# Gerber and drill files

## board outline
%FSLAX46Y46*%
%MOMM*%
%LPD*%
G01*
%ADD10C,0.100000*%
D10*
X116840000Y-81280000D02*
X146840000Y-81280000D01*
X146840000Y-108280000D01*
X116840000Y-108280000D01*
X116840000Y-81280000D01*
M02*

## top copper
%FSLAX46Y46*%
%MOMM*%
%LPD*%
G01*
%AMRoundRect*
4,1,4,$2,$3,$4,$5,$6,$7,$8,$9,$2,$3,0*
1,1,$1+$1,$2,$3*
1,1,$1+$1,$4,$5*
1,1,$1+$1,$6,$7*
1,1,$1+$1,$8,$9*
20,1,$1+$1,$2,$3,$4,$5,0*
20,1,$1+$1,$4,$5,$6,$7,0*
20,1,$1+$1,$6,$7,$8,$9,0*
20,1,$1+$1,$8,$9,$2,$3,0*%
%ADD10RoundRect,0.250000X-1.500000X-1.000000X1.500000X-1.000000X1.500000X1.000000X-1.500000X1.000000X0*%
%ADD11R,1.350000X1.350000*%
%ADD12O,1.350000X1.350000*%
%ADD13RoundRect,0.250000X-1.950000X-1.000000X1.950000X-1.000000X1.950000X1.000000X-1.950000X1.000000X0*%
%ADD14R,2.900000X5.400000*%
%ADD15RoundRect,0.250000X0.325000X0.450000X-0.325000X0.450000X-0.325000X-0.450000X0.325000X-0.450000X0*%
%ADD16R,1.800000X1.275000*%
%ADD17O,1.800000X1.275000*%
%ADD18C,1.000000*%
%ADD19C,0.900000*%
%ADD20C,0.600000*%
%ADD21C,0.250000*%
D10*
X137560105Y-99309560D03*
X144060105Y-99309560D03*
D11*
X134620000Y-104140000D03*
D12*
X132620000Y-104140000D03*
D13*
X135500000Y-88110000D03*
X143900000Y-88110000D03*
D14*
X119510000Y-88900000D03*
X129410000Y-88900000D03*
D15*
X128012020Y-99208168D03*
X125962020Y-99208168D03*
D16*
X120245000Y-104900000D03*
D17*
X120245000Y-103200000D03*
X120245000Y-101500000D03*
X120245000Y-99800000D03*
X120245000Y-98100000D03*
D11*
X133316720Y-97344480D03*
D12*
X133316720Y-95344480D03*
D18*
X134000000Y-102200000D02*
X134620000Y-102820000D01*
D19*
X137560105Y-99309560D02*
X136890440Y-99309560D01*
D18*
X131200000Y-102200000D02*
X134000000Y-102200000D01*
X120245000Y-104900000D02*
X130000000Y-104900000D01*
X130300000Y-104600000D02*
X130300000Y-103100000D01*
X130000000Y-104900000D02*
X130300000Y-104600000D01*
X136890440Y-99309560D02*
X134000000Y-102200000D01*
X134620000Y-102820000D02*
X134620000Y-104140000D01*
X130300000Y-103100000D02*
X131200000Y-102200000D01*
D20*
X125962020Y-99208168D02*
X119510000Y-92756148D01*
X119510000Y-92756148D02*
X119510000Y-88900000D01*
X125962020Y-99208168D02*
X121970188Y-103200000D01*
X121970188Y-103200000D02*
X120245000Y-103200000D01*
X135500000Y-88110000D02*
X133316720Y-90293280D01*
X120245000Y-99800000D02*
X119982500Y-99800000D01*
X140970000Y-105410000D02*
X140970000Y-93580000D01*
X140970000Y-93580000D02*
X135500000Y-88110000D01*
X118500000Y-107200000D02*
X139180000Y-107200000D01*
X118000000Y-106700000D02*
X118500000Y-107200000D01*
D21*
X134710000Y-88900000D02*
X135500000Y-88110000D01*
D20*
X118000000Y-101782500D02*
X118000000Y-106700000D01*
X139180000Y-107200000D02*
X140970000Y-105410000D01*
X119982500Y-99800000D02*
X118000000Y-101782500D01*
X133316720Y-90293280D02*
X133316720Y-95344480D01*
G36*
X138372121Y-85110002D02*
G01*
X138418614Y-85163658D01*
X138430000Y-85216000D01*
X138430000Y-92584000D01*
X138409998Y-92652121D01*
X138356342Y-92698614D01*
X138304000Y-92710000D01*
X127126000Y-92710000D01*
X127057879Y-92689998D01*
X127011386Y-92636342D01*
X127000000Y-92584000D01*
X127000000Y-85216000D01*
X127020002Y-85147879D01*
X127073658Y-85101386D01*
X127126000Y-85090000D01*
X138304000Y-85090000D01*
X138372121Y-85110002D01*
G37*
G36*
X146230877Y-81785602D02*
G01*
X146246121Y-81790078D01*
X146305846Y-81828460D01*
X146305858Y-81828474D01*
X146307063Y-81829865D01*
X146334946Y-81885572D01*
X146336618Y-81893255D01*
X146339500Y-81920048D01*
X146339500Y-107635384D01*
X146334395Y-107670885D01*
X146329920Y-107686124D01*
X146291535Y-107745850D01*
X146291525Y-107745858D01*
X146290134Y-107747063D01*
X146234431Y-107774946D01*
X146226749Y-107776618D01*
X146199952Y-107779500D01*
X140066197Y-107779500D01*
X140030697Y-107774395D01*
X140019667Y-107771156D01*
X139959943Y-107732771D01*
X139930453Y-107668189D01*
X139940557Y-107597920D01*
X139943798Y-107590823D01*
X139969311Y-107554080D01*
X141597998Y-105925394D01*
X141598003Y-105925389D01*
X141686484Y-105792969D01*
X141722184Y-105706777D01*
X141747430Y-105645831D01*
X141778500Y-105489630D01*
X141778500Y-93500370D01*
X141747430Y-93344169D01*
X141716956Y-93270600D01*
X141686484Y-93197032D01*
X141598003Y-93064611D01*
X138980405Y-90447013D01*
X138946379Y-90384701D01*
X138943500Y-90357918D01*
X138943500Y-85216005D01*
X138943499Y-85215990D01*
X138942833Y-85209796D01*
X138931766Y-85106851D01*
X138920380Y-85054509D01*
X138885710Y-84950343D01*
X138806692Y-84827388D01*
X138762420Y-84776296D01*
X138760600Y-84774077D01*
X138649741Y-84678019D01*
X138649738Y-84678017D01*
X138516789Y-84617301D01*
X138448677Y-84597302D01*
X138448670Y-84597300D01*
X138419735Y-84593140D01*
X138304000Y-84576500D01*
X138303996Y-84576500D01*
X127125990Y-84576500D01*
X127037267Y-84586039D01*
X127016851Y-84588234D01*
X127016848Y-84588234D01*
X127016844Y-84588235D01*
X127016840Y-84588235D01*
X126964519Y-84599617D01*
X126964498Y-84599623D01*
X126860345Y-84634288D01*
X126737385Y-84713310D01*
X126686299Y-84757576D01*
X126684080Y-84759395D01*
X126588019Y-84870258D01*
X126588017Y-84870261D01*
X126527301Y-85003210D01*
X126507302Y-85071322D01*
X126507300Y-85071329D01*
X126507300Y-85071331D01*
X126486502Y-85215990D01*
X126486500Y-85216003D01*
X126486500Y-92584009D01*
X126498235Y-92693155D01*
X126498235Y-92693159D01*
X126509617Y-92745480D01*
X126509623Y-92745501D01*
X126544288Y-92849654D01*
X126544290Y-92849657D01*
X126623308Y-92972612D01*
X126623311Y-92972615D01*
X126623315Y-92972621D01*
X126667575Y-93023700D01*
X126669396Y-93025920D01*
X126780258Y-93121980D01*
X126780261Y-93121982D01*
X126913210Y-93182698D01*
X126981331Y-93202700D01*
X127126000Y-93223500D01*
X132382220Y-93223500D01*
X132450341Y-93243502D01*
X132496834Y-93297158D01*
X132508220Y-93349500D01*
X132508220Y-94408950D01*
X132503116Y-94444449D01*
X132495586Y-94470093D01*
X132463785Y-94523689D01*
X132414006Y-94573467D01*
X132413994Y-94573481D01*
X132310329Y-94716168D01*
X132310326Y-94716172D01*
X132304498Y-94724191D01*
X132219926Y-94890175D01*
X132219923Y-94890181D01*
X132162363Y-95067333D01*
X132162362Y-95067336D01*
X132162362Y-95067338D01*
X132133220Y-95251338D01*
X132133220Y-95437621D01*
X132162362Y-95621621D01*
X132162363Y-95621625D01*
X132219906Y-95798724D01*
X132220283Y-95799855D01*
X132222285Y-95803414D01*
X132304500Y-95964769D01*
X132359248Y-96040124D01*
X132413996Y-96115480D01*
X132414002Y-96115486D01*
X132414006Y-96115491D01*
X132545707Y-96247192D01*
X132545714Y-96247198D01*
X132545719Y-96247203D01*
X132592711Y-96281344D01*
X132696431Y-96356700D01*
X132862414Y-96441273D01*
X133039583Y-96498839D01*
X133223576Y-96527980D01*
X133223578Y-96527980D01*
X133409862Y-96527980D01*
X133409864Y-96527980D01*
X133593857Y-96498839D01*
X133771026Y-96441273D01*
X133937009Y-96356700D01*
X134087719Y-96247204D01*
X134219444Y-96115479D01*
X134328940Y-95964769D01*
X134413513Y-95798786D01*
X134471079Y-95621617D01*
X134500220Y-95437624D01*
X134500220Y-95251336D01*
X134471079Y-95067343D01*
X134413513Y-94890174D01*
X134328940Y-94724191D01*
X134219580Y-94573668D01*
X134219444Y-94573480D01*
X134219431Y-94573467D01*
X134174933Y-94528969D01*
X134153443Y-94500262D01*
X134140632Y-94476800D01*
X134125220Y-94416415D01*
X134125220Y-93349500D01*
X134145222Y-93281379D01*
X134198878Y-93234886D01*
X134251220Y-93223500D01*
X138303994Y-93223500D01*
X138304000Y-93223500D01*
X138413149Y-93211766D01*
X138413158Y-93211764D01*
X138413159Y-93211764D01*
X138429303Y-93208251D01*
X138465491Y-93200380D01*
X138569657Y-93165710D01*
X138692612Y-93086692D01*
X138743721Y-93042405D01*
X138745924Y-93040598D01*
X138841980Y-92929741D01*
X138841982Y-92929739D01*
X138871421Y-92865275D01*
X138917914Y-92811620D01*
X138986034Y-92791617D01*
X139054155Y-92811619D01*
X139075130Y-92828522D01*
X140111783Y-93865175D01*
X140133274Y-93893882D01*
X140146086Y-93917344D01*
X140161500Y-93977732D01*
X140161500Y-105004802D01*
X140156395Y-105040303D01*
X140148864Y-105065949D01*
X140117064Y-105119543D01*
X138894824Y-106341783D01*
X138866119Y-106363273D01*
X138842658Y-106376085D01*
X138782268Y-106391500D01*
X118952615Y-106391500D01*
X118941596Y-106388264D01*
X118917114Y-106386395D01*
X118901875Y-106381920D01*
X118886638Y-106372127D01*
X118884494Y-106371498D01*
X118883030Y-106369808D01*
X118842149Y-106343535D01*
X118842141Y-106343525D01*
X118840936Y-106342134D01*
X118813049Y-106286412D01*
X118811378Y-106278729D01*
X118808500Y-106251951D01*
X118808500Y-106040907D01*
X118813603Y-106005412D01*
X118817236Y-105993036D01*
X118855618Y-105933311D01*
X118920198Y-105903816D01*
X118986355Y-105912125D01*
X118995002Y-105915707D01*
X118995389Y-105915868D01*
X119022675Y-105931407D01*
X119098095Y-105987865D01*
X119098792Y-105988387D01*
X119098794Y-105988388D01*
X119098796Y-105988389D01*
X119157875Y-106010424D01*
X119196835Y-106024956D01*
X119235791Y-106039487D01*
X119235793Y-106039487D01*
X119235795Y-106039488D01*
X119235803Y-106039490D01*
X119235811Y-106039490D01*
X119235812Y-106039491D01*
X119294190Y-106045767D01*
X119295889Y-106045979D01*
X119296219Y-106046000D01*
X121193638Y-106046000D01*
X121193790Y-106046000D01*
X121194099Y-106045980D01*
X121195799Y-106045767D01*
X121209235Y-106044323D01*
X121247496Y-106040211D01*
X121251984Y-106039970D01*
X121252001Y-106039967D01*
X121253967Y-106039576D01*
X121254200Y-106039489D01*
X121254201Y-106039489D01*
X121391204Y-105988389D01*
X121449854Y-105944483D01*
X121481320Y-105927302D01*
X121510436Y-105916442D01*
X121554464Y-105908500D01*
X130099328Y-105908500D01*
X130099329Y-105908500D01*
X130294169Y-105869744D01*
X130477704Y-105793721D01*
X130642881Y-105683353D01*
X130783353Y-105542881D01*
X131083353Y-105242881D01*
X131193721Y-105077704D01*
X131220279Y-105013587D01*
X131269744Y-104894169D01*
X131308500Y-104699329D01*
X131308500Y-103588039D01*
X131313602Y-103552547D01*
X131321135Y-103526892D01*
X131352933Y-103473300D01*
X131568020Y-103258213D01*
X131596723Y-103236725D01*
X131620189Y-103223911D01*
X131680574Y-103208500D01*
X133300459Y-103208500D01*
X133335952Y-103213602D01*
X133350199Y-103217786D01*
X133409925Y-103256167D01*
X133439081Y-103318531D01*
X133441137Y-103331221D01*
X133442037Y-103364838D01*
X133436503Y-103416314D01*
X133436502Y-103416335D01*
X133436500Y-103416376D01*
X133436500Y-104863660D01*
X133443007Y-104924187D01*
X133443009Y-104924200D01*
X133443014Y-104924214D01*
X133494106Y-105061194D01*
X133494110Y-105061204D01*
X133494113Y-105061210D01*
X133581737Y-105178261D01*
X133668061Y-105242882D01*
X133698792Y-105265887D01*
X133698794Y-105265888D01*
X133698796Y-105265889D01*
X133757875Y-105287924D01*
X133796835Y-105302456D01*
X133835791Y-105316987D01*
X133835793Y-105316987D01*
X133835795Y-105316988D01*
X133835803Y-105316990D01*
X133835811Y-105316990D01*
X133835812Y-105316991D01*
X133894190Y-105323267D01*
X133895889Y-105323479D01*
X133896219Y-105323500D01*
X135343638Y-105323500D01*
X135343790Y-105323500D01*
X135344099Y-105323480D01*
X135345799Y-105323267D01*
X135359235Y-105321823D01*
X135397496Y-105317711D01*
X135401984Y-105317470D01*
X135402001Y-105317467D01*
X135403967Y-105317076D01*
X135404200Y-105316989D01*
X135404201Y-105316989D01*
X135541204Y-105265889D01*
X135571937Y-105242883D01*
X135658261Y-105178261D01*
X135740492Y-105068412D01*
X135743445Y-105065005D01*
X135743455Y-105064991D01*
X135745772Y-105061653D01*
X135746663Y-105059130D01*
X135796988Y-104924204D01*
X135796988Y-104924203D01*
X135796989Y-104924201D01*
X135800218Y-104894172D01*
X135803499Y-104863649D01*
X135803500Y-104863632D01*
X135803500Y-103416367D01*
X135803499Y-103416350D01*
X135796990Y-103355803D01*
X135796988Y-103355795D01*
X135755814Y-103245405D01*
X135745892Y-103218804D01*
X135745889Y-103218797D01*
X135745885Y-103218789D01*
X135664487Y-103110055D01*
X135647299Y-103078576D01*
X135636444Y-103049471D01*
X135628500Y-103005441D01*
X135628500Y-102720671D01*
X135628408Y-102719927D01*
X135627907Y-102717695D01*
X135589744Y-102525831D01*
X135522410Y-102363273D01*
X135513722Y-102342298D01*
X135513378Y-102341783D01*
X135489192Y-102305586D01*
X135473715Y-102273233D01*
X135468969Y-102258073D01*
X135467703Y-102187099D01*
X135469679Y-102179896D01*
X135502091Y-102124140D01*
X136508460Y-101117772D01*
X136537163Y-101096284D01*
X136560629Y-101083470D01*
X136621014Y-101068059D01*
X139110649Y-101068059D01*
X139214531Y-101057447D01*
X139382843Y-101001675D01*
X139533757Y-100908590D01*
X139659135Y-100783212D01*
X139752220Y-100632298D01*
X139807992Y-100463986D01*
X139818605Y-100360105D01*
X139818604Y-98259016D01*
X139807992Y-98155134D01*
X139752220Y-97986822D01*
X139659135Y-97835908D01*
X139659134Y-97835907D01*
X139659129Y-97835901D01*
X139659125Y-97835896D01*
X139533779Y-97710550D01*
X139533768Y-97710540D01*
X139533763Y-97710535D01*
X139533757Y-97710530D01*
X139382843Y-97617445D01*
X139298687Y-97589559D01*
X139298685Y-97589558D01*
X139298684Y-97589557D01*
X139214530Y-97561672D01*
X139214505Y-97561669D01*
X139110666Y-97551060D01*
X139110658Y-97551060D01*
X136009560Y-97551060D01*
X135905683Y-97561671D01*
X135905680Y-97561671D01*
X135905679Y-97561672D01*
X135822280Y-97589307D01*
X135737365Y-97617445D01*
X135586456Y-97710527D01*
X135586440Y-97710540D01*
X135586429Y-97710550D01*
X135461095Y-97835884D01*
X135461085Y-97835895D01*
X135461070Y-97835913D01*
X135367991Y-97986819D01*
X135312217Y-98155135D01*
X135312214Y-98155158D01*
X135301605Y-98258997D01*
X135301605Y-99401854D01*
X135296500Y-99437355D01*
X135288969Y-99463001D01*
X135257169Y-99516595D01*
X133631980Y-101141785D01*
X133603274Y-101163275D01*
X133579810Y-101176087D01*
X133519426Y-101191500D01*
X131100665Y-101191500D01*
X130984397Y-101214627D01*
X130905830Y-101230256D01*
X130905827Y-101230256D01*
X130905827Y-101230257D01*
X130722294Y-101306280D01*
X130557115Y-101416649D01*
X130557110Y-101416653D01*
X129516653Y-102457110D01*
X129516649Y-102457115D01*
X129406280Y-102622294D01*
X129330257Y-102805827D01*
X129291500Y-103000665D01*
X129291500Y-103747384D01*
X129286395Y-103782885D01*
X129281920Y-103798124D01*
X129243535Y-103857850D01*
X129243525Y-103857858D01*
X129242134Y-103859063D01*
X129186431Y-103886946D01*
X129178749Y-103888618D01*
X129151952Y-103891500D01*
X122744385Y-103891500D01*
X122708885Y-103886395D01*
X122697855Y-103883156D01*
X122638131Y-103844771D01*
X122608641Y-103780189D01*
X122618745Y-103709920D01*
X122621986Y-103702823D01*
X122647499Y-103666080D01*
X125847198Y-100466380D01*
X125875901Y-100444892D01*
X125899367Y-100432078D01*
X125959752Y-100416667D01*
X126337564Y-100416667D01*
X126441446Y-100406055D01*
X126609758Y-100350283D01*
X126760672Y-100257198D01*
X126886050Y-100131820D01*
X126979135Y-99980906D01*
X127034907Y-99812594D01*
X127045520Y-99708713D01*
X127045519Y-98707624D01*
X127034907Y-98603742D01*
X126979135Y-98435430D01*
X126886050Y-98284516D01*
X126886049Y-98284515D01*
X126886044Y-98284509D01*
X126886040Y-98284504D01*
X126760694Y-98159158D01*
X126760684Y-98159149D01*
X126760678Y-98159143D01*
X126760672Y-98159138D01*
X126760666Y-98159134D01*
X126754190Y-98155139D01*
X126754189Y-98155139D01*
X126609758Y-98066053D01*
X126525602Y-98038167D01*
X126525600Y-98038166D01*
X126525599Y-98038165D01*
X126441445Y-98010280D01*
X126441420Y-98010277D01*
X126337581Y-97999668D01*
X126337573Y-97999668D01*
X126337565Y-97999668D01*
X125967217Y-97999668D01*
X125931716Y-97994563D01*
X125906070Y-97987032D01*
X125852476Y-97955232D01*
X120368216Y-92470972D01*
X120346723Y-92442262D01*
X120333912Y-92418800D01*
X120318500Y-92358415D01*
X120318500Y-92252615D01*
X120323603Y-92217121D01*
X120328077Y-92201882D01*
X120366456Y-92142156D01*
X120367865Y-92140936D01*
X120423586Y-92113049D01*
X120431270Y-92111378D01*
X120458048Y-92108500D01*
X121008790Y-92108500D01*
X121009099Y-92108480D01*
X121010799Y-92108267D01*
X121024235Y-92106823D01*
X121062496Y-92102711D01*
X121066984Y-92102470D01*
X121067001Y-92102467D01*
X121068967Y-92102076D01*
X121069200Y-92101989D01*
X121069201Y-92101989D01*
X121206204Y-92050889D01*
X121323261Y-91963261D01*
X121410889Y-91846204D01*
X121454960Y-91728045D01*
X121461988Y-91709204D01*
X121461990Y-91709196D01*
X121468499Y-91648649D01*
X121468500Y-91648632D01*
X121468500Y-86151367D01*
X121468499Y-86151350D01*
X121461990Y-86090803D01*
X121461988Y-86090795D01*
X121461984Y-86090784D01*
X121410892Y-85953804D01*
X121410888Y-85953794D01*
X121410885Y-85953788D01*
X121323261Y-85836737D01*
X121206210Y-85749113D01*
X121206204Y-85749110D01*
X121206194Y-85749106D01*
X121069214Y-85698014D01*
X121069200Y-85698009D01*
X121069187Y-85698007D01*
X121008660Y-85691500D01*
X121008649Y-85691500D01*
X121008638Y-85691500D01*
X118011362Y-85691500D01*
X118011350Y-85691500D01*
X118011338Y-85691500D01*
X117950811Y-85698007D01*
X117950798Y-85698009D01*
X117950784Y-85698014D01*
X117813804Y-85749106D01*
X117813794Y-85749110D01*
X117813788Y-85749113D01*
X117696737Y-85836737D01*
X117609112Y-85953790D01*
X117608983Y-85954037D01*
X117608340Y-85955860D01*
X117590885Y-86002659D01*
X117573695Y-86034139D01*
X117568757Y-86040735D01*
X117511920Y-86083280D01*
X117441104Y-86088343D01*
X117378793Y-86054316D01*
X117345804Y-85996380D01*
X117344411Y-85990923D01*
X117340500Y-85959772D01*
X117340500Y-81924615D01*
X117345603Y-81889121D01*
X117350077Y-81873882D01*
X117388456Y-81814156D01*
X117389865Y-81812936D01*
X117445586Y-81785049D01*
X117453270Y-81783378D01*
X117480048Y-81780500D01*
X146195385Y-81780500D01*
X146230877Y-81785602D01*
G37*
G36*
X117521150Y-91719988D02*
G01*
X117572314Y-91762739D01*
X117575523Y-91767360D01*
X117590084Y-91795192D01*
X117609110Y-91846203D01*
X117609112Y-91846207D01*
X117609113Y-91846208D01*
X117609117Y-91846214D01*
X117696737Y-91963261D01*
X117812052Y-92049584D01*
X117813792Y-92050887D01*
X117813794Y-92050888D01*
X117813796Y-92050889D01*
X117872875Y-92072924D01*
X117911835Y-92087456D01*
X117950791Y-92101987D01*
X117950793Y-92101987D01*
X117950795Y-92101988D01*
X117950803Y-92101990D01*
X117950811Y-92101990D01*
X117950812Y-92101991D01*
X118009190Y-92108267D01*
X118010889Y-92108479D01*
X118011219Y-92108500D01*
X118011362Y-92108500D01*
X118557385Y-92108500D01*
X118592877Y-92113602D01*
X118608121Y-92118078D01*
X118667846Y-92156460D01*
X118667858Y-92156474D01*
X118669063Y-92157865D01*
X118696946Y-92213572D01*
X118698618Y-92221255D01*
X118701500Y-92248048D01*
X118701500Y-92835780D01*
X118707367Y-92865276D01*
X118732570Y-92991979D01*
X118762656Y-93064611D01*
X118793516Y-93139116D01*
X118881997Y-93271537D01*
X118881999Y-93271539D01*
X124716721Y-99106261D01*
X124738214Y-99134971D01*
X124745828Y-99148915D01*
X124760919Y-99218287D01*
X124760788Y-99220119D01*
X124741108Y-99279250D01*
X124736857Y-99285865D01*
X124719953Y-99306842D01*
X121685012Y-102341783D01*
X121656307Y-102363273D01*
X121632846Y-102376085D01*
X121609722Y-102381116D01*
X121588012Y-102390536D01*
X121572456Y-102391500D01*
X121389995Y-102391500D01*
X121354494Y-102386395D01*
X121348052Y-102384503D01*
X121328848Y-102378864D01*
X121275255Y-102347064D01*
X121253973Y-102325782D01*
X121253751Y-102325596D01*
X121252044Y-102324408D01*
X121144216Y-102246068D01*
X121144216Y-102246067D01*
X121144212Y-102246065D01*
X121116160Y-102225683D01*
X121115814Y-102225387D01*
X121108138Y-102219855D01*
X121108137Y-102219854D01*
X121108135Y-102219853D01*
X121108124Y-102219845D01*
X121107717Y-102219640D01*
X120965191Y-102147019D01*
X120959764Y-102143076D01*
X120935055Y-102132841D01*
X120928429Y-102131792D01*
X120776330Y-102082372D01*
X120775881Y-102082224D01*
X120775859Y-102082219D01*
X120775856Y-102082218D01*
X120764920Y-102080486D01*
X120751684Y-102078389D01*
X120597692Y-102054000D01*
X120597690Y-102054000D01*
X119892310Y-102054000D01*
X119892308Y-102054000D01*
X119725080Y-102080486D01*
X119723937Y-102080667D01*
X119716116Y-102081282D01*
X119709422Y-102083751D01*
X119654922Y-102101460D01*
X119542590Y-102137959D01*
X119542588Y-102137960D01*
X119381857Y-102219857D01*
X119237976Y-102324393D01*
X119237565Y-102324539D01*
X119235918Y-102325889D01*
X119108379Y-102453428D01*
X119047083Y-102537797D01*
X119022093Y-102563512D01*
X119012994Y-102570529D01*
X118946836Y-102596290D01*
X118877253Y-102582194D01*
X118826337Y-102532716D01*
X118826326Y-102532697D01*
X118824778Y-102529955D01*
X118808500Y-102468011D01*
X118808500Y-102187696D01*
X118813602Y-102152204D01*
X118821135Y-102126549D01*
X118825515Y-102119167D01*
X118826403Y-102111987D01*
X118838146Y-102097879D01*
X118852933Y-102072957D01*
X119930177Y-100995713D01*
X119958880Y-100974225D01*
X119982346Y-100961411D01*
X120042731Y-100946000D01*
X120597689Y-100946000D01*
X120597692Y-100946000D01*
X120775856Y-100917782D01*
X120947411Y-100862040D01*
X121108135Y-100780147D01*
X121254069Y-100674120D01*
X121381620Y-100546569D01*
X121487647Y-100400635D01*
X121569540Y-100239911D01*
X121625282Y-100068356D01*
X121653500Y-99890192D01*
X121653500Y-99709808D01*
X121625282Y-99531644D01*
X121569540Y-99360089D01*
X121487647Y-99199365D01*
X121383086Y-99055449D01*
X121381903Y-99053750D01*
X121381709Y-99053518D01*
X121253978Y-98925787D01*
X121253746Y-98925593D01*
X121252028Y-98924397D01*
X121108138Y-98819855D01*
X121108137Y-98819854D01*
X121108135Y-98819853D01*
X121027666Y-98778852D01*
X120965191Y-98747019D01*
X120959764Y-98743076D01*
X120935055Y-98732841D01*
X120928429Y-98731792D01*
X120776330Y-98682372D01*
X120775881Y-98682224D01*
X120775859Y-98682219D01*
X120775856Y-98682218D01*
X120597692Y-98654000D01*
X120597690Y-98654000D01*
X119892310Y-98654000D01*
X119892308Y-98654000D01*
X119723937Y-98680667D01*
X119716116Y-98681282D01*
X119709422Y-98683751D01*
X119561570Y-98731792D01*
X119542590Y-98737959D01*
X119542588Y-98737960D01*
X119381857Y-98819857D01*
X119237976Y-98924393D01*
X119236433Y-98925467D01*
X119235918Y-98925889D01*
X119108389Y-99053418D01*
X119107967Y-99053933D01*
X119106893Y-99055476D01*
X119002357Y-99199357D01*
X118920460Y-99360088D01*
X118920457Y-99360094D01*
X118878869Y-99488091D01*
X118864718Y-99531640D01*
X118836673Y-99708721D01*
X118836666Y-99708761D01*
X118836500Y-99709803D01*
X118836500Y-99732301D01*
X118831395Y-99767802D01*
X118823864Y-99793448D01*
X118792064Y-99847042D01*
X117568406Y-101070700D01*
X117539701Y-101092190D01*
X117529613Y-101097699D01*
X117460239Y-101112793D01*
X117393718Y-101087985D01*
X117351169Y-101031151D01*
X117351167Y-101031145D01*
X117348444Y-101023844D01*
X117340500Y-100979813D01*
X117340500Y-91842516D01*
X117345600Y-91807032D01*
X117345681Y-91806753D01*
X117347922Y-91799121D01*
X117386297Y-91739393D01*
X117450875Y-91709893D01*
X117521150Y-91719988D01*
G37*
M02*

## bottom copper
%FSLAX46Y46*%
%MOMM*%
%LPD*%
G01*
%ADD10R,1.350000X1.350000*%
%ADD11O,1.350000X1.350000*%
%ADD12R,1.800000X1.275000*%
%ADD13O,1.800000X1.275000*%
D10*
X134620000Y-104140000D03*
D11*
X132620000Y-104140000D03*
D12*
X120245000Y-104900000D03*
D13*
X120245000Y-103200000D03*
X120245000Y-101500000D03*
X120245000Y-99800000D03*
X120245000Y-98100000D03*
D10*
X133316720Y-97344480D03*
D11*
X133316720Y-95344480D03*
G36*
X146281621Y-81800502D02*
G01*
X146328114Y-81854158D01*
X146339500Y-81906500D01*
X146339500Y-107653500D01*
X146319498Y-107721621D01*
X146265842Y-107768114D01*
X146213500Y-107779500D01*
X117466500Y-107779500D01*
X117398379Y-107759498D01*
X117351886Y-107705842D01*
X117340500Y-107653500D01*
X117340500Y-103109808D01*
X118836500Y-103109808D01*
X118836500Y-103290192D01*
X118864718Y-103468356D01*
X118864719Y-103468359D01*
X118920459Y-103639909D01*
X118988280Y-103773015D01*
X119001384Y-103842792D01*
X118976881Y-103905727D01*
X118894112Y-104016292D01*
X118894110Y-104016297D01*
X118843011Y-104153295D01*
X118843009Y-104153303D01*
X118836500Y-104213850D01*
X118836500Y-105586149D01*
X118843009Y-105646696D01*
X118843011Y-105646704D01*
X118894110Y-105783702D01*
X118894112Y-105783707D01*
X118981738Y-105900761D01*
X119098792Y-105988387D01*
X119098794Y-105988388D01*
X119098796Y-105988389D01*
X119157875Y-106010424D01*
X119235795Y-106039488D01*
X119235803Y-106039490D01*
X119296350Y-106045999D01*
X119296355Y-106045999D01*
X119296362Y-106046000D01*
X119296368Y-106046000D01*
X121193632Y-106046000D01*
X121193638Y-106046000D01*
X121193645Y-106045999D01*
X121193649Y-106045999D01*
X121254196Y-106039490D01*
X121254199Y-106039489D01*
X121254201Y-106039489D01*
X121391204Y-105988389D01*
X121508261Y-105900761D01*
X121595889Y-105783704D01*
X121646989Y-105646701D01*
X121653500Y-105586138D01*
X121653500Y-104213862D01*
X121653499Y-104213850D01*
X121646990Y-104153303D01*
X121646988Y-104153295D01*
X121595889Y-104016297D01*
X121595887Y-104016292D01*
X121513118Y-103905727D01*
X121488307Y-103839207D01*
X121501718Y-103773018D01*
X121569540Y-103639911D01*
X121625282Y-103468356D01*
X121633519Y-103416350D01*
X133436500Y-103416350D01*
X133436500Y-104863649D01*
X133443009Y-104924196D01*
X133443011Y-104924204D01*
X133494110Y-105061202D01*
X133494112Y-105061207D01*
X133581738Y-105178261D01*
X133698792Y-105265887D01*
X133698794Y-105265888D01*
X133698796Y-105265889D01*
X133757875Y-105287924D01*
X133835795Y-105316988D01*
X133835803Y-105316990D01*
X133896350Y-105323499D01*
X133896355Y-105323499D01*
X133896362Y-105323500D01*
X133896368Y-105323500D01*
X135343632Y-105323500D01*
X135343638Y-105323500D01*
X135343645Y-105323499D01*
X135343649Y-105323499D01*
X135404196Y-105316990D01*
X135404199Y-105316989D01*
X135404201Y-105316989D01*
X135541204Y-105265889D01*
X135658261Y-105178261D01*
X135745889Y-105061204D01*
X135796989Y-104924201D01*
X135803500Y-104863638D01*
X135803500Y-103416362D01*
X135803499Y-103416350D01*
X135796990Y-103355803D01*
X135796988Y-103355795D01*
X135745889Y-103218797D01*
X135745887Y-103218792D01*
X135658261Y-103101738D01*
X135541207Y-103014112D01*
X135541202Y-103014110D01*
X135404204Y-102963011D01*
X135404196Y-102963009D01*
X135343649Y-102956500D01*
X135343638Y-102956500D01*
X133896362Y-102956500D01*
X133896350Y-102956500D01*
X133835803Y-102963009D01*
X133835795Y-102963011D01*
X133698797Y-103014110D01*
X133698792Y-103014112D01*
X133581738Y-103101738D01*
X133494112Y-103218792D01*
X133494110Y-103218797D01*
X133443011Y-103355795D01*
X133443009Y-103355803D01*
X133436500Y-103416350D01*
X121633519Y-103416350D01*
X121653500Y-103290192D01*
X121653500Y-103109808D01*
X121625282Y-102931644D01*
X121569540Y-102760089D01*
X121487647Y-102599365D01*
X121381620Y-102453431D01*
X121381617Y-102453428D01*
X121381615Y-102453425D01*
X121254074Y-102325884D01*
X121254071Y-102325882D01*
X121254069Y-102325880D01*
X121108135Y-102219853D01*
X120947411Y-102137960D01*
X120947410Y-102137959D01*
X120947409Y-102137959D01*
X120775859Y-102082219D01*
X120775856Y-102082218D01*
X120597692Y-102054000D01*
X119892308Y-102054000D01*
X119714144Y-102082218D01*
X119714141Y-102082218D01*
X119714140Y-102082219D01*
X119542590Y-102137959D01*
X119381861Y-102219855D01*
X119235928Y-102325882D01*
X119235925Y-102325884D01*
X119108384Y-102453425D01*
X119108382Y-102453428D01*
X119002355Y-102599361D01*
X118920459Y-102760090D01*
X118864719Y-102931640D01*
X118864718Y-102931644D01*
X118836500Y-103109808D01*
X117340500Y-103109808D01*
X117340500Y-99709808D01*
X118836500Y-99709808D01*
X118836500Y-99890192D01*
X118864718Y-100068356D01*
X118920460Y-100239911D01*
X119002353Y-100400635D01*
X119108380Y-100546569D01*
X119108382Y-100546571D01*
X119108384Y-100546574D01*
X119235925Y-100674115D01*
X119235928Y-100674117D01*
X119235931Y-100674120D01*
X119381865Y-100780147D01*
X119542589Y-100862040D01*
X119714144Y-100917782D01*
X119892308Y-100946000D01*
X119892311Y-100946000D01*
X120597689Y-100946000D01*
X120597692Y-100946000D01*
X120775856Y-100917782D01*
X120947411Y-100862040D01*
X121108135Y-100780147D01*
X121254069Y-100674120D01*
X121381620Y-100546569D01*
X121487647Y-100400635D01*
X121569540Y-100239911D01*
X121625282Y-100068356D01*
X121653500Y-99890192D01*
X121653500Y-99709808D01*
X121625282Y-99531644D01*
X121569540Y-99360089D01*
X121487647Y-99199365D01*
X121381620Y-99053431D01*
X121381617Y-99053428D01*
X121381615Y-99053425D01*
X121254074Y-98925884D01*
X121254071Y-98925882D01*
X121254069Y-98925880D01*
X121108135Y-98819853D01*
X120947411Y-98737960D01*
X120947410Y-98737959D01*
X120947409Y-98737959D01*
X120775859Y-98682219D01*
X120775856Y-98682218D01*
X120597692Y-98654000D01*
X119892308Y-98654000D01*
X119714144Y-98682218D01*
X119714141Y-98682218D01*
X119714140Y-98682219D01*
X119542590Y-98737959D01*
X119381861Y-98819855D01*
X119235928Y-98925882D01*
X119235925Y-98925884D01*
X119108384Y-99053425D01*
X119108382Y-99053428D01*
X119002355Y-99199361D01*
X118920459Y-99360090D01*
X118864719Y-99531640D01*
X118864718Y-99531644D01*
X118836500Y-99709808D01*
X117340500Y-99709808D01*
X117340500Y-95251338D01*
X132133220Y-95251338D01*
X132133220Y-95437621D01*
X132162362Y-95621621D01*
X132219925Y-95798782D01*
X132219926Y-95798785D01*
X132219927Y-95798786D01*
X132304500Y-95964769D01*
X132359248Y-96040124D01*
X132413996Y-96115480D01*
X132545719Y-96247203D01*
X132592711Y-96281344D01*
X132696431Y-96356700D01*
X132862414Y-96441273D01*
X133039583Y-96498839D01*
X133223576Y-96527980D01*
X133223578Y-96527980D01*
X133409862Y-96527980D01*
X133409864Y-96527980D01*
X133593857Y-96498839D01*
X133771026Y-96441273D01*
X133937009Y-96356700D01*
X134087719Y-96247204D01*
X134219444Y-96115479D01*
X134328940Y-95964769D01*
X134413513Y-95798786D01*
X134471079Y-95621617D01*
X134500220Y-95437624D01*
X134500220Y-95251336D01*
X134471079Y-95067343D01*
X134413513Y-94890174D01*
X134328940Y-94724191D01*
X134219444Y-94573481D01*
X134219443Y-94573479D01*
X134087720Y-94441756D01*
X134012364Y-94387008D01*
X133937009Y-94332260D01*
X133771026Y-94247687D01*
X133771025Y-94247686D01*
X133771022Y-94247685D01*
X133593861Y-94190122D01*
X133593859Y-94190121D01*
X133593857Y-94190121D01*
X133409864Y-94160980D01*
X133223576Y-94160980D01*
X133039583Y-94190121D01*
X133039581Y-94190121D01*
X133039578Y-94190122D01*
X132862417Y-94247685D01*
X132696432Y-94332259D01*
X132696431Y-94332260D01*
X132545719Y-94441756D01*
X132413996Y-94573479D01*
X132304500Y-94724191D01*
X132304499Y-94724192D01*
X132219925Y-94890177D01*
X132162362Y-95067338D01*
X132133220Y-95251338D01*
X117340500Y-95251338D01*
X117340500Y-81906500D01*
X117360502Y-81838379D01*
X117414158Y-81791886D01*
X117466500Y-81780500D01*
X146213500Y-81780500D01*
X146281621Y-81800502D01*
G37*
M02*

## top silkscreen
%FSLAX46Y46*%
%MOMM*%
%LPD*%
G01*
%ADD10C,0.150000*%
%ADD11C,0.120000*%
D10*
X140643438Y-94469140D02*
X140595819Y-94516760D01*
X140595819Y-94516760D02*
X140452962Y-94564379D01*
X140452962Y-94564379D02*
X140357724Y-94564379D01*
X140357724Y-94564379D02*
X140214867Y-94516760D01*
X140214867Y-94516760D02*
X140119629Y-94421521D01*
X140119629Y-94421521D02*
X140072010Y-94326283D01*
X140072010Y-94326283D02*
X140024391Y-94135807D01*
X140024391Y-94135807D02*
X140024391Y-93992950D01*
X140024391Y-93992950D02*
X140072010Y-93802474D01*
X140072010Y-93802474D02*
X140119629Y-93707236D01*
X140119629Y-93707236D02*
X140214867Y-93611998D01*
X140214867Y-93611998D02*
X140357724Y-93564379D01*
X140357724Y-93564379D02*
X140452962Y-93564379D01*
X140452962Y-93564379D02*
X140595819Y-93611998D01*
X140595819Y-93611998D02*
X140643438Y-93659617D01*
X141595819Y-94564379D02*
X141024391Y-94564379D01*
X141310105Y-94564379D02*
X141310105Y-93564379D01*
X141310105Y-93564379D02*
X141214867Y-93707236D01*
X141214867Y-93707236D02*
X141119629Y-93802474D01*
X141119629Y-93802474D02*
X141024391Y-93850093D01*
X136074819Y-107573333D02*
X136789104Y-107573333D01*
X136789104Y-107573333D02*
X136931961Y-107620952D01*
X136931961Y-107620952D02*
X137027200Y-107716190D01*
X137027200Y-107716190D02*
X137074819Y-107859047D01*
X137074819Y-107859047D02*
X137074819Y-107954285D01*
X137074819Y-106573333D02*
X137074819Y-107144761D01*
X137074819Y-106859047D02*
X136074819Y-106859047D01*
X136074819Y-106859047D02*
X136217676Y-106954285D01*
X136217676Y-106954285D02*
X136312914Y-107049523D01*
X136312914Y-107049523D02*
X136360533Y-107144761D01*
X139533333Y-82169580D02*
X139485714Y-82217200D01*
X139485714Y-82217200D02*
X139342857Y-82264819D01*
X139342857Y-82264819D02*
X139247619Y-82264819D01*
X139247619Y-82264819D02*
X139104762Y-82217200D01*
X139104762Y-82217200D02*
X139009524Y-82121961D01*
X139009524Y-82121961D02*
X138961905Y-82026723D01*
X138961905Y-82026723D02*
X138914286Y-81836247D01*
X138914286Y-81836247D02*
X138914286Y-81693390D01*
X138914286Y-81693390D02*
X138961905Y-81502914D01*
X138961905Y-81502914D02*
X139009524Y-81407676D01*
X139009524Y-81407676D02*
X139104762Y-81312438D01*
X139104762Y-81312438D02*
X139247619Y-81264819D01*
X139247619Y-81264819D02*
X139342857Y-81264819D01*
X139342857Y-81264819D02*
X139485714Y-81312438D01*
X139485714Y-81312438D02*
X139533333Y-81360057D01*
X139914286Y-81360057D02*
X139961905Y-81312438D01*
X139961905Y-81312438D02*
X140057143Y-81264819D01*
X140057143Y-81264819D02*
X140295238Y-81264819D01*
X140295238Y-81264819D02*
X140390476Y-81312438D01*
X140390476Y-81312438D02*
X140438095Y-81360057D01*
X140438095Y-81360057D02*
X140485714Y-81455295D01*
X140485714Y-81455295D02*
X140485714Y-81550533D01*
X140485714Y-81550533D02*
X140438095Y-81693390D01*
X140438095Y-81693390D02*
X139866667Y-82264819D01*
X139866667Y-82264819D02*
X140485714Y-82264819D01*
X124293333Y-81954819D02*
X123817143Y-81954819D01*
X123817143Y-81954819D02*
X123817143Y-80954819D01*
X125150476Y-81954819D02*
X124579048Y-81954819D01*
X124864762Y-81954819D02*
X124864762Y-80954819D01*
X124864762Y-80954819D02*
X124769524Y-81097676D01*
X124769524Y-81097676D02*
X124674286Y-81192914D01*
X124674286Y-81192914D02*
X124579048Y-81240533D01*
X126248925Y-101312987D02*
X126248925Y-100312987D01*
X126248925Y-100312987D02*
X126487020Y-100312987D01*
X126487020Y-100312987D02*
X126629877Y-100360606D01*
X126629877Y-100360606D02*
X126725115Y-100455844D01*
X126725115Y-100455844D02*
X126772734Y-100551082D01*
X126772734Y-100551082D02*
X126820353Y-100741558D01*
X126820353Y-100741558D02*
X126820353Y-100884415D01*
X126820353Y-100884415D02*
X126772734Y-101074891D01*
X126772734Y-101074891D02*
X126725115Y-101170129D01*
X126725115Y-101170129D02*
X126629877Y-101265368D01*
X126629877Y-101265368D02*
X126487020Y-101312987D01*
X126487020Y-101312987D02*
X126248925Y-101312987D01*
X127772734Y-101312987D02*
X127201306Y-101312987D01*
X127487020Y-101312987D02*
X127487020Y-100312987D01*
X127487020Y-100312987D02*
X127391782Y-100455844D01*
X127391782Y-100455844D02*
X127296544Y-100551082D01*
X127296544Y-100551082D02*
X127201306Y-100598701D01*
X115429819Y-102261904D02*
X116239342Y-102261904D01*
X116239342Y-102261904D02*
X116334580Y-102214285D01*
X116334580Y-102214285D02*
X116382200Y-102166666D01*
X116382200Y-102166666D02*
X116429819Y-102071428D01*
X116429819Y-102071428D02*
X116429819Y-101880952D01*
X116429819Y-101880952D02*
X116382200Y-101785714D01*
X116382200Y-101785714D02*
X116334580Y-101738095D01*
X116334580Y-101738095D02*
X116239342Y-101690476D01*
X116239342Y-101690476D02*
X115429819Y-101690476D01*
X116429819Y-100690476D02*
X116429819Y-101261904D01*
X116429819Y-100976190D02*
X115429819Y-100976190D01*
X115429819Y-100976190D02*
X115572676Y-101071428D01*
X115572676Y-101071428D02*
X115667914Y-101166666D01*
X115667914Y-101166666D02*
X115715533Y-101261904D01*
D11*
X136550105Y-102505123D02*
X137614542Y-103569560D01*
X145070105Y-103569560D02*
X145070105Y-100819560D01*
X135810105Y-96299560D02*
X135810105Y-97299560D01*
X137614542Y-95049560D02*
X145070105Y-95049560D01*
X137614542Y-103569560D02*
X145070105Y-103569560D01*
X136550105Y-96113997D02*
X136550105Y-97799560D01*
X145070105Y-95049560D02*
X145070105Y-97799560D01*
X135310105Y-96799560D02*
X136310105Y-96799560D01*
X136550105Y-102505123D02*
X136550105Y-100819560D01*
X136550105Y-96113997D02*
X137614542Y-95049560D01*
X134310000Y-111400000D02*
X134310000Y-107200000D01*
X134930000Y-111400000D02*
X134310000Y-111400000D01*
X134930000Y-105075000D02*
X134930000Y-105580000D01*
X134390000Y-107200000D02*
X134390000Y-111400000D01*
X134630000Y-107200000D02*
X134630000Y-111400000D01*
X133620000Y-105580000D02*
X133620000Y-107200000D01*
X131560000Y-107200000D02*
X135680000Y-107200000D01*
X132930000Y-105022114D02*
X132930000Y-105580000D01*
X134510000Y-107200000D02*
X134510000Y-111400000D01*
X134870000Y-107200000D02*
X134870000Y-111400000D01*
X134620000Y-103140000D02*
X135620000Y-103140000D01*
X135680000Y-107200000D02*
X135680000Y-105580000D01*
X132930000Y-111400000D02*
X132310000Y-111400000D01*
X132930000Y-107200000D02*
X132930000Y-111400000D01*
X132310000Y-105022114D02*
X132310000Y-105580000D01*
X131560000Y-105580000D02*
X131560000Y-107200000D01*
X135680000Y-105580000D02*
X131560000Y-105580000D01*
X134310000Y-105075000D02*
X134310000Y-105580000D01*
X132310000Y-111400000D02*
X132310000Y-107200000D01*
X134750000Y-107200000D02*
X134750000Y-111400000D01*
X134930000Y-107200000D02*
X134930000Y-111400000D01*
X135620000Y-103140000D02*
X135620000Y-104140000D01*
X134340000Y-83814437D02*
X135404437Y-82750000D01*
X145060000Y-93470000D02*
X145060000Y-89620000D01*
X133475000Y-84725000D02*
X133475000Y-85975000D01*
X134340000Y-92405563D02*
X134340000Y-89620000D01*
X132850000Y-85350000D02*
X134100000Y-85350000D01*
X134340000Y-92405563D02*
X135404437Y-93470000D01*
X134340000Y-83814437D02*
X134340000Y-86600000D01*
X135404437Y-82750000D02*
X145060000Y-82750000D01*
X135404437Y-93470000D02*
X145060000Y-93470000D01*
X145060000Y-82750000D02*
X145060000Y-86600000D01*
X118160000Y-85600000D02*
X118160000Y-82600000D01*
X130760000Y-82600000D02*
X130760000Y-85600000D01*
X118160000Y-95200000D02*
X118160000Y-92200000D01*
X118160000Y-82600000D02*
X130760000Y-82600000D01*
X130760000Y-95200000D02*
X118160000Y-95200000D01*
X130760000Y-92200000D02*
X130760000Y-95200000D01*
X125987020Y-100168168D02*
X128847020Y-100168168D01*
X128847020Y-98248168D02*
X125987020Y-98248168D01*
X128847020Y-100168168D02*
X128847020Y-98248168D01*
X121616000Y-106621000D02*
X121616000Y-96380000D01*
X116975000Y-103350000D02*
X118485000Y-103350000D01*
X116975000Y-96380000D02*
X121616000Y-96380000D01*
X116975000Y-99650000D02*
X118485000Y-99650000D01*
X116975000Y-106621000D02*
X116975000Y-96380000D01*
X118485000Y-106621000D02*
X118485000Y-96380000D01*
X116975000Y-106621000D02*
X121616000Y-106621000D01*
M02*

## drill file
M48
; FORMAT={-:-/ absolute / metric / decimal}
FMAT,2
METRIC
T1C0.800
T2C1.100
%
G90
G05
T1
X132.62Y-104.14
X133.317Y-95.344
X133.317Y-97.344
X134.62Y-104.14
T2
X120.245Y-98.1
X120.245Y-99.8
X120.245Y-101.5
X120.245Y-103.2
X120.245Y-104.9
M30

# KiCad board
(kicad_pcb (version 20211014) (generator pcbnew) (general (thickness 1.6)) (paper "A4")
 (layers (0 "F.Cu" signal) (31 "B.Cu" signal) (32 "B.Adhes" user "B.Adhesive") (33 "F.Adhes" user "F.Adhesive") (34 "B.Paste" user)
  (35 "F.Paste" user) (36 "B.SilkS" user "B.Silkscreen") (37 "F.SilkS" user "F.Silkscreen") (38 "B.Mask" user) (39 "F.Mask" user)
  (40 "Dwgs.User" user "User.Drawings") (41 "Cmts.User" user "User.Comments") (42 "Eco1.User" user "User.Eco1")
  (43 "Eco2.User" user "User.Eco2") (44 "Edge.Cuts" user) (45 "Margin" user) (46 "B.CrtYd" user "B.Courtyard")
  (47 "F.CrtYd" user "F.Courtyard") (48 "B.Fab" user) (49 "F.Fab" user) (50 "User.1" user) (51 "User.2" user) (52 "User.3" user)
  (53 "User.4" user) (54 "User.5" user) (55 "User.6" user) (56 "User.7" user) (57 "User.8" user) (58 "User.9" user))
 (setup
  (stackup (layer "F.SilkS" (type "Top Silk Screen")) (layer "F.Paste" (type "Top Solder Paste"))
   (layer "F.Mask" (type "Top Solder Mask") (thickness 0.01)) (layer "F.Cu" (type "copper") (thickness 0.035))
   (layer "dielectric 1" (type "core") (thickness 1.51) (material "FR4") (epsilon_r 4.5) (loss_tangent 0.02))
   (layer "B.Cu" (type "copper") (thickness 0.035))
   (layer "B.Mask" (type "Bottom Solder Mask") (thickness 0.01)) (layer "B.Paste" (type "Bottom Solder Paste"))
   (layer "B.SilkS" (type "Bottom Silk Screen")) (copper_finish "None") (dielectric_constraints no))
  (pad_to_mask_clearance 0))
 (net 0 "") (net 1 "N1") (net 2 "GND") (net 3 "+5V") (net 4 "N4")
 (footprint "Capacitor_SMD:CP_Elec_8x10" (layer "F.Cu") (at 140.810105 99.30956)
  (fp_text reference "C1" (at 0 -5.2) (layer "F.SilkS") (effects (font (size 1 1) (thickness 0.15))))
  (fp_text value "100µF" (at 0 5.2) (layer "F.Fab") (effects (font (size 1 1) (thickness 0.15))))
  (fp_line (start -4.26 3.195563) (end -3.195563 4.26) (layer "F.SilkS") (width 0.12))
  (fp_line (start 4.26 4.26) (end 4.26 1.51) (layer "F.SilkS") (width 0.12))
  (fp_line (start -5 -3.01) (end -5 -2.01) (layer "F.SilkS") (width 0.12))
  (fp_line (start -3.195563 -4.26) (end 4.26 -4.26) (layer "F.SilkS") (width 0.12))
  (fp_line (start -3.195563 4.26) (end 4.26 4.26) (layer "F.SilkS") (width 0.12))
  (fp_line (start -4.26 -3.195563) (end -4.26 -1.51) (layer "F.SilkS") (width 0.12))
  (fp_line (start 4.26 -4.26) (end 4.26 -1.51) (layer "F.SilkS") (width 0.12))
  (fp_line (start -5.5 -2.51) (end -4.5 -2.51) (layer "F.SilkS") (width 0.12))
  (fp_line (start -4.26 3.195563) (end -4.26 1.51) (layer "F.SilkS") (width 0.12))
  (fp_line (start -4.26 -3.195563) (end -3.195563 -4.26) (layer "F.SilkS") (width 0.12))
  (pad "1" smd roundrect (at -3.25 0) (size 3.5 2.5) (layers "F.Cu" "F.Paste" "F.Mask") (roundrect_rratio 0.1) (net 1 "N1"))
  (pad "2" smd roundrect (at 3.25 0) (size 3.5 2.5) (layers "F.Cu" "F.Paste" "F.Mask") (roundrect_rratio 0.1) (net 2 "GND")))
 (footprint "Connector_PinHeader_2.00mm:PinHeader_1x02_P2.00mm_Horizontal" (layer "F.Cu") (at 134.62 104.14 -90)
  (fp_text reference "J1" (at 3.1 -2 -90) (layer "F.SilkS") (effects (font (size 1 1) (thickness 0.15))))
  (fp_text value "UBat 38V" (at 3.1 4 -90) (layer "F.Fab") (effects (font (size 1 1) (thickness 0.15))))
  (fp_line (start 7.26 0.31) (end 3.06 0.31) (layer "F.SilkS") (width 0.12))
  (fp_line (start 7.26 -0.31) (end 7.26 0.31) (layer "F.SilkS") (width 0.12))
  (fp_line (start 0.935 -0.31) (end 1.44 -0.31) (layer "F.SilkS") (width 0.12))
  (fp_line (start 3.06 0.23) (end 7.26 0.23) (layer "F.SilkS") (width 0.12))
  (fp_line (start 3.06 -0.01) (end 7.26 -0.01) (layer "F.SilkS") (width 0.12))
  (fp_line (start 1.44 1) (end 3.06 1) (layer "F.SilkS") (width 0.12))
  (fp_line (start 3.06 3.06) (end 3.06 -1.06) (layer "F.SilkS") (width 0.12))
  (fp_line (start 0.882114 1.69) (end 1.44 1.69) (layer "F.SilkS") (width 0.12))
  (fp_line (start 3.06 0.11) (end 7.26 0.11) (layer "F.SilkS") (width 0.12))
  (fp_line (start 3.06 -0.25) (end 7.26 -0.25) (layer "F.SilkS") (width 0.12))
  (fp_line (start -1 0) (end -1 -1) (layer "F.SilkS") (width 0.12))
  (fp_line (start 3.06 -1.06) (end 1.44 -1.06) (layer "F.SilkS") (width 0.12))
  (fp_line (start 7.26 1.69) (end 7.26 2.31) (layer "F.SilkS") (width 0.12))
  (fp_line (start 3.06 1.69) (end 7.26 1.69) (layer "F.SilkS") (width 0.12))
  (fp_line (start 0.882114 2.31) (end 1.44 2.31) (layer "F.SilkS") (width 0.12))
  (fp_line (start 1.44 3.06) (end 3.06 3.06) (layer "F.SilkS") (width 0.12))
  (fp_line (start 1.44 -1.06) (end 1.44 3.06) (layer "F.SilkS") (width 0.12))
  (fp_line (start 0.935 0.31) (end 1.44 0.31) (layer "F.SilkS") (width 0.12))
  (fp_line (start 7.26 2.31) (end 3.06 2.31) (layer "F.SilkS") (width 0.12))
  (fp_line (start 3.06 -0.13) (end 7.26 -0.13) (layer "F.SilkS") (width 0.12))
  (fp_line (start 3.06 -0.31) (end 7.26 -0.31) (layer "F.SilkS") (width 0.12))
  (fp_line (start -1 -1) (end 0 -1) (layer "F.SilkS") (width 0.12))
  (pad "1" thru_hole rect (at 0 0 270) (size 1.35 1.35) (drill 0.8) (layers *.Cu *.Mask) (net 1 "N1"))
  (pad "2" thru_hole oval (at 0 2 270) (size 1.35 1.35) (drill 0.8) (layers *.Cu *.Mask) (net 2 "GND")))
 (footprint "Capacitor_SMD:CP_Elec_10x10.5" (layer "F.Cu") (at 139.7 88.11)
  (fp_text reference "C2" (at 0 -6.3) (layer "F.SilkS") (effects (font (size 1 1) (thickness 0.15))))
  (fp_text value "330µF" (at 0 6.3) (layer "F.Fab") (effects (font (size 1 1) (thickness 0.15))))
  (fp_line (start -5.36 -4.295563) (end -4.295563 -5.36) (layer "F.SilkS") (width 0.12))
  (fp_line (start 5.36 5.36) (end 5.36 1.51) (layer "F.SilkS") (width 0.12))
  (fp_line (start -6.225 -3.385) (end -6.225 -2.135) (layer "F.SilkS") (width 0.12))
  (fp_line (start -5.36 4.295563) (end -5.36 1.51) (layer "F.SilkS") (width 0.12))
  (fp_line (start -6.85 -2.76) (end -5.6 -2.76) (layer "F.SilkS") (width 0.12))
  (fp_line (start -5.36 4.295563) (end -4.295563 5.36) (layer "F.SilkS") (width 0.12))
  (fp_line (start -5.36 -4.295563) (end -5.36 -1.51) (layer "F.SilkS") (width 0.12))
  (fp_line (start -4.295563 -5.36) (end 5.36 -5.36) (layer "F.SilkS") (width 0.12))
  (fp_line (start -4.295563 5.36) (end 5.36 5.36) (layer "F.SilkS") (width 0.12))
  (fp_line (start 5.36 -5.36) (end 5.36 -1.51) (layer "F.SilkS") (width 0.12))
  (pad "1" smd roundrect (at -4.2 0) (size 4.4 2.5) (layers "F.Cu" "F.Paste" "F.Mask") (roundrect_rratio 0.1) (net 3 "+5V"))
  (pad "2" smd roundrect (at 4.2 0) (size 4.4 2.5) (layers "F.Cu" "F.Paste" "F.Mask") (roundrect_rratio 0.1) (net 2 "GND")))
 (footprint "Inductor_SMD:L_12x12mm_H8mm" (layer "F.Cu") (at 124.46 88.9)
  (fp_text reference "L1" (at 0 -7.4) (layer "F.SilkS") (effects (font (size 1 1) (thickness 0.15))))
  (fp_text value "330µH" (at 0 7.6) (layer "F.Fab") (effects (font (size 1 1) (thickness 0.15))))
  (fp_line (start -6.3 -3.3) (end -6.3 -6.3) (layer "F.SilkS") (width 0.12))
  (fp_line (start 6.3 -6.3) (end 6.3 -3.3) (layer "F.SilkS") (width 0.12))
  (fp_line (start -6.3 6.3) (end -6.3 3.3) (layer "F.SilkS") (width 0.12))
  (fp_line (start -6.3 -6.3) (end 6.3 -6.3) (layer "F.SilkS") (width 0.12))
  (fp_line (start 6.3 6.3) (end -6.3 6.3) (layer "F.SilkS") (width 0.12))
  (fp_line (start 6.3 3.3) (end 6.3 6.3) (layer "F.SilkS") (width 0.12))
  (pad "1" smd rect (at -4.95 0) (size 2.9 5.4) (layers "F.Cu" "F.Paste" "F.Mask") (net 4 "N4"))
  (pad "2" smd rect (at 4.95 0) (size 2.9 5.4) (layers "F.Cu" "F.Paste" "F.Mask") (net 3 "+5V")))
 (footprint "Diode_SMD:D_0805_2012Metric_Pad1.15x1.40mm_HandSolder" (layer "F.Cu") (at 126.98702 99.208168 180)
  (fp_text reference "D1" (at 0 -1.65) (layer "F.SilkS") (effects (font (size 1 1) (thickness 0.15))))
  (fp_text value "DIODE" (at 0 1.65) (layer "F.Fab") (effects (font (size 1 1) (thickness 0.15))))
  (fp_line (start 1 -0.96) (end -1.86 -0.96) (layer "F.SilkS") (width 0.12))
  (fp_line (start -1.86 0.96) (end 1 0.96) (layer "F.SilkS") (width 0.12))
  (fp_line (start -1.86 -0.96) (end -1.86 0.96) (layer "F.SilkS") (width 0.12))
  (pad "1" smd roundrect (at -1.025 0 180) (size 1.15 1.4) (layers "F.Cu" "F.Paste" "F.Mask") (roundrect_rratio 0.217391) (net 2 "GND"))
  (pad "2" smd roundrect (at 1.025 0 180) (size 1.15 1.4) (layers "F.Cu" "F.Paste" "F.Mask") (roundrect_rratio 0.217391) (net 4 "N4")))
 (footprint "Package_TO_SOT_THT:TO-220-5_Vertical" (layer "F.Cu") (at 120.245 104.9 90)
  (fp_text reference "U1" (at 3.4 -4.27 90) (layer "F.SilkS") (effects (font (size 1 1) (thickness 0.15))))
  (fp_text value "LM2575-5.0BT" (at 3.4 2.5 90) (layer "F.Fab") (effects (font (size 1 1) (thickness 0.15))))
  (fp_line (start -1.721 1.371) (end 8.52 1.371) (layer "F.SilkS") (width 0.12))
  (fp_line (start 1.55 -3.27) (end 1.55 -1.76) (layer "F.SilkS") (width 0.12))
  (fp_line (start 8.52 -3.27) (end 8.52 1.371) (layer "F.SilkS") (width 0.12))
  (fp_line (start 5.25 -3.27) (end 5.25 -1.76) (layer "F.SilkS") (width 0.12))
  (fp_line (start -1.721 -3.27) (end 8.52 -3.27) (layer "F.SilkS") (width 0.12))
  (fp_line (start -1.721 -1.76) (end 8.52 -1.76) (layer "F.SilkS") (width 0.12))
  (fp_line (start -1.721 -3.27) (end -1.721 1.371) (layer "F.SilkS") (width 0.12))
  (pad "1" thru_hole rect (at 0 0 90) (size 1.275 1.8) (drill 1.1) (layers *.Cu *.Mask) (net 1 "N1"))
  (pad "2" thru_hole oval (at 1.7 0 90) (size 1.275 1.8) (drill 1.1) (layers *.Cu *.Mask) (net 4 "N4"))
  (pad "3" thru_hole oval (at 3.4 0 90) (size 1.275 1.8) (drill 1.1) (layers *.Cu *.Mask) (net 2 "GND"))
  (pad "4" thru_hole oval (at 5.1 0 90) (size 1.275 1.8) (drill 1.1) (layers *.Cu *.Mask) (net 3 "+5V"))
  (pad "5" thru_hole oval (at 6.8 0 90) (size 1.275 1.8) (drill 1.1) (layers *.Cu *.Mask) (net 2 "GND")))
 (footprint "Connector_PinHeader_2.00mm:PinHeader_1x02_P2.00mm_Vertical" (layer "B.Cu") (at 133.31672 97.34448)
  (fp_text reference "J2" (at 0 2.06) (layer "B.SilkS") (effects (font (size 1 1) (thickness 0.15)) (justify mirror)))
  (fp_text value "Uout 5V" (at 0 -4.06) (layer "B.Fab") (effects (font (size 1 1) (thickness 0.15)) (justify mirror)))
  (pad "1" thru_hole rect (at 0 0) (size 1.35 1.35) (drill 0.8) (layers *.Cu *.Mask) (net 2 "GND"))
  (pad "2" thru_hole oval (at 0 -2) (size 1.35 1.35) (drill 0.8) (layers *.Cu *.Mask) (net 3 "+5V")))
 (gr_rect (start 116.84 81.28) (end 146.84 108.28) (layer "Edge.Cuts") (width 0.1) (fill none))
 (segment (start 134 102.2) (end 134.62 102.82) (width 1) (layer "F.Cu") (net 1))
 (segment (start 137.560105 99.30956) (end 136.89044 99.30956) (width 0.9) (layer "F.Cu") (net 1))
 (segment (start 131.2 102.2) (end 134 102.2) (width 1) (layer "F.Cu") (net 1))
 (segment (start 120.245 104.9) (end 130 104.9) (width 1) (layer "F.Cu") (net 1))
 (segment (start 130.3 104.6) (end 130.3 103.1) (width 1) (layer "F.Cu") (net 1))
 (segment (start 130 104.9) (end 130.3 104.6) (width 1) (layer "F.Cu") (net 1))
 (segment (start 136.89044 99.30956) (end 134 102.2) (width 1) (layer "F.Cu") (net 1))
 (segment (start 134.62 102.82) (end 134.62 104.14) (width 1) (layer "F.Cu") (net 1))
 (segment (start 130.3 103.1) (end 131.2 102.2) (width 1) (layer "F.Cu") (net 1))
 (segment (start 125.96202 99.208168) (end 119.51 92.756148) (width 0.6) (layer "F.Cu") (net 4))
 (segment (start 119.51 92.756148) (end 119.51 88.9) (width 0.6) (layer "F.Cu") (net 4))
 (segment (start 125.96202 99.208168) (end 121.970188 103.2) (width 0.6) (layer "F.Cu") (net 4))
 (segment (start 121.970188 103.2) (end 120.245 103.2) (width 0.6) (layer "F.Cu") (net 4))
 (segment (start 135.5 88.11) (end 133.31672 90.29328) (width 0.6) (layer "F.Cu") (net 3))
 (segment (start 120.245 99.8) (end 119.9825 99.8) (width 0.6) (layer "F.Cu") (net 3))
 (segment (start 140.97 105.41) (end 140.97 93.58) (width 0.6) (layer "F.Cu") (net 3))
 (segment (start 140.97 93.58) (end 135.5 88.11) (width 0.6) (layer "F.Cu") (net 3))
 (segment (start 118.5 107.2) (end 139.18 107.2) (width 0.6) (layer "F.Cu") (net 3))
 (segment (start 118 106.7) (end 118.5 107.2) (width 0.6) (layer "F.Cu") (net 3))
 (segment (start 134.71 88.9) (end 135.5 88.11) (width 0.25) (layer "F.Cu") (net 3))
 (segment (start 118 101.7825) (end 118 106.7) (width 0.6) (layer "F.Cu") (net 3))
 (segment (start 139.18 107.2) (end 140.97 105.41) (width 0.6) (layer "F.Cu") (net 3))
 (segment (start 119.9825 99.8) (end 118 101.7825) (width 0.6) (layer "F.Cu") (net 3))
 (segment (start 133.31672 90.29328) (end 133.31672 95.34448) (width 0.6) (layer "F.Cu") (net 3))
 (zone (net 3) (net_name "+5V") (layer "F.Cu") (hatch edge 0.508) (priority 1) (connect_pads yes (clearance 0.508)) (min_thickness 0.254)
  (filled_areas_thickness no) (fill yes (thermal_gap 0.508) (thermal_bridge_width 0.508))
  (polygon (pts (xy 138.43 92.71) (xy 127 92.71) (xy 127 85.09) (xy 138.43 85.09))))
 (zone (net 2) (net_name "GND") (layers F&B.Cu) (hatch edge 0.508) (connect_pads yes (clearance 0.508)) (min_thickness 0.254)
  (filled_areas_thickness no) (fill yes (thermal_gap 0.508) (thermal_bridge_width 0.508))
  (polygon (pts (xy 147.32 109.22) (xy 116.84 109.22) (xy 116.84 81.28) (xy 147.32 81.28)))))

